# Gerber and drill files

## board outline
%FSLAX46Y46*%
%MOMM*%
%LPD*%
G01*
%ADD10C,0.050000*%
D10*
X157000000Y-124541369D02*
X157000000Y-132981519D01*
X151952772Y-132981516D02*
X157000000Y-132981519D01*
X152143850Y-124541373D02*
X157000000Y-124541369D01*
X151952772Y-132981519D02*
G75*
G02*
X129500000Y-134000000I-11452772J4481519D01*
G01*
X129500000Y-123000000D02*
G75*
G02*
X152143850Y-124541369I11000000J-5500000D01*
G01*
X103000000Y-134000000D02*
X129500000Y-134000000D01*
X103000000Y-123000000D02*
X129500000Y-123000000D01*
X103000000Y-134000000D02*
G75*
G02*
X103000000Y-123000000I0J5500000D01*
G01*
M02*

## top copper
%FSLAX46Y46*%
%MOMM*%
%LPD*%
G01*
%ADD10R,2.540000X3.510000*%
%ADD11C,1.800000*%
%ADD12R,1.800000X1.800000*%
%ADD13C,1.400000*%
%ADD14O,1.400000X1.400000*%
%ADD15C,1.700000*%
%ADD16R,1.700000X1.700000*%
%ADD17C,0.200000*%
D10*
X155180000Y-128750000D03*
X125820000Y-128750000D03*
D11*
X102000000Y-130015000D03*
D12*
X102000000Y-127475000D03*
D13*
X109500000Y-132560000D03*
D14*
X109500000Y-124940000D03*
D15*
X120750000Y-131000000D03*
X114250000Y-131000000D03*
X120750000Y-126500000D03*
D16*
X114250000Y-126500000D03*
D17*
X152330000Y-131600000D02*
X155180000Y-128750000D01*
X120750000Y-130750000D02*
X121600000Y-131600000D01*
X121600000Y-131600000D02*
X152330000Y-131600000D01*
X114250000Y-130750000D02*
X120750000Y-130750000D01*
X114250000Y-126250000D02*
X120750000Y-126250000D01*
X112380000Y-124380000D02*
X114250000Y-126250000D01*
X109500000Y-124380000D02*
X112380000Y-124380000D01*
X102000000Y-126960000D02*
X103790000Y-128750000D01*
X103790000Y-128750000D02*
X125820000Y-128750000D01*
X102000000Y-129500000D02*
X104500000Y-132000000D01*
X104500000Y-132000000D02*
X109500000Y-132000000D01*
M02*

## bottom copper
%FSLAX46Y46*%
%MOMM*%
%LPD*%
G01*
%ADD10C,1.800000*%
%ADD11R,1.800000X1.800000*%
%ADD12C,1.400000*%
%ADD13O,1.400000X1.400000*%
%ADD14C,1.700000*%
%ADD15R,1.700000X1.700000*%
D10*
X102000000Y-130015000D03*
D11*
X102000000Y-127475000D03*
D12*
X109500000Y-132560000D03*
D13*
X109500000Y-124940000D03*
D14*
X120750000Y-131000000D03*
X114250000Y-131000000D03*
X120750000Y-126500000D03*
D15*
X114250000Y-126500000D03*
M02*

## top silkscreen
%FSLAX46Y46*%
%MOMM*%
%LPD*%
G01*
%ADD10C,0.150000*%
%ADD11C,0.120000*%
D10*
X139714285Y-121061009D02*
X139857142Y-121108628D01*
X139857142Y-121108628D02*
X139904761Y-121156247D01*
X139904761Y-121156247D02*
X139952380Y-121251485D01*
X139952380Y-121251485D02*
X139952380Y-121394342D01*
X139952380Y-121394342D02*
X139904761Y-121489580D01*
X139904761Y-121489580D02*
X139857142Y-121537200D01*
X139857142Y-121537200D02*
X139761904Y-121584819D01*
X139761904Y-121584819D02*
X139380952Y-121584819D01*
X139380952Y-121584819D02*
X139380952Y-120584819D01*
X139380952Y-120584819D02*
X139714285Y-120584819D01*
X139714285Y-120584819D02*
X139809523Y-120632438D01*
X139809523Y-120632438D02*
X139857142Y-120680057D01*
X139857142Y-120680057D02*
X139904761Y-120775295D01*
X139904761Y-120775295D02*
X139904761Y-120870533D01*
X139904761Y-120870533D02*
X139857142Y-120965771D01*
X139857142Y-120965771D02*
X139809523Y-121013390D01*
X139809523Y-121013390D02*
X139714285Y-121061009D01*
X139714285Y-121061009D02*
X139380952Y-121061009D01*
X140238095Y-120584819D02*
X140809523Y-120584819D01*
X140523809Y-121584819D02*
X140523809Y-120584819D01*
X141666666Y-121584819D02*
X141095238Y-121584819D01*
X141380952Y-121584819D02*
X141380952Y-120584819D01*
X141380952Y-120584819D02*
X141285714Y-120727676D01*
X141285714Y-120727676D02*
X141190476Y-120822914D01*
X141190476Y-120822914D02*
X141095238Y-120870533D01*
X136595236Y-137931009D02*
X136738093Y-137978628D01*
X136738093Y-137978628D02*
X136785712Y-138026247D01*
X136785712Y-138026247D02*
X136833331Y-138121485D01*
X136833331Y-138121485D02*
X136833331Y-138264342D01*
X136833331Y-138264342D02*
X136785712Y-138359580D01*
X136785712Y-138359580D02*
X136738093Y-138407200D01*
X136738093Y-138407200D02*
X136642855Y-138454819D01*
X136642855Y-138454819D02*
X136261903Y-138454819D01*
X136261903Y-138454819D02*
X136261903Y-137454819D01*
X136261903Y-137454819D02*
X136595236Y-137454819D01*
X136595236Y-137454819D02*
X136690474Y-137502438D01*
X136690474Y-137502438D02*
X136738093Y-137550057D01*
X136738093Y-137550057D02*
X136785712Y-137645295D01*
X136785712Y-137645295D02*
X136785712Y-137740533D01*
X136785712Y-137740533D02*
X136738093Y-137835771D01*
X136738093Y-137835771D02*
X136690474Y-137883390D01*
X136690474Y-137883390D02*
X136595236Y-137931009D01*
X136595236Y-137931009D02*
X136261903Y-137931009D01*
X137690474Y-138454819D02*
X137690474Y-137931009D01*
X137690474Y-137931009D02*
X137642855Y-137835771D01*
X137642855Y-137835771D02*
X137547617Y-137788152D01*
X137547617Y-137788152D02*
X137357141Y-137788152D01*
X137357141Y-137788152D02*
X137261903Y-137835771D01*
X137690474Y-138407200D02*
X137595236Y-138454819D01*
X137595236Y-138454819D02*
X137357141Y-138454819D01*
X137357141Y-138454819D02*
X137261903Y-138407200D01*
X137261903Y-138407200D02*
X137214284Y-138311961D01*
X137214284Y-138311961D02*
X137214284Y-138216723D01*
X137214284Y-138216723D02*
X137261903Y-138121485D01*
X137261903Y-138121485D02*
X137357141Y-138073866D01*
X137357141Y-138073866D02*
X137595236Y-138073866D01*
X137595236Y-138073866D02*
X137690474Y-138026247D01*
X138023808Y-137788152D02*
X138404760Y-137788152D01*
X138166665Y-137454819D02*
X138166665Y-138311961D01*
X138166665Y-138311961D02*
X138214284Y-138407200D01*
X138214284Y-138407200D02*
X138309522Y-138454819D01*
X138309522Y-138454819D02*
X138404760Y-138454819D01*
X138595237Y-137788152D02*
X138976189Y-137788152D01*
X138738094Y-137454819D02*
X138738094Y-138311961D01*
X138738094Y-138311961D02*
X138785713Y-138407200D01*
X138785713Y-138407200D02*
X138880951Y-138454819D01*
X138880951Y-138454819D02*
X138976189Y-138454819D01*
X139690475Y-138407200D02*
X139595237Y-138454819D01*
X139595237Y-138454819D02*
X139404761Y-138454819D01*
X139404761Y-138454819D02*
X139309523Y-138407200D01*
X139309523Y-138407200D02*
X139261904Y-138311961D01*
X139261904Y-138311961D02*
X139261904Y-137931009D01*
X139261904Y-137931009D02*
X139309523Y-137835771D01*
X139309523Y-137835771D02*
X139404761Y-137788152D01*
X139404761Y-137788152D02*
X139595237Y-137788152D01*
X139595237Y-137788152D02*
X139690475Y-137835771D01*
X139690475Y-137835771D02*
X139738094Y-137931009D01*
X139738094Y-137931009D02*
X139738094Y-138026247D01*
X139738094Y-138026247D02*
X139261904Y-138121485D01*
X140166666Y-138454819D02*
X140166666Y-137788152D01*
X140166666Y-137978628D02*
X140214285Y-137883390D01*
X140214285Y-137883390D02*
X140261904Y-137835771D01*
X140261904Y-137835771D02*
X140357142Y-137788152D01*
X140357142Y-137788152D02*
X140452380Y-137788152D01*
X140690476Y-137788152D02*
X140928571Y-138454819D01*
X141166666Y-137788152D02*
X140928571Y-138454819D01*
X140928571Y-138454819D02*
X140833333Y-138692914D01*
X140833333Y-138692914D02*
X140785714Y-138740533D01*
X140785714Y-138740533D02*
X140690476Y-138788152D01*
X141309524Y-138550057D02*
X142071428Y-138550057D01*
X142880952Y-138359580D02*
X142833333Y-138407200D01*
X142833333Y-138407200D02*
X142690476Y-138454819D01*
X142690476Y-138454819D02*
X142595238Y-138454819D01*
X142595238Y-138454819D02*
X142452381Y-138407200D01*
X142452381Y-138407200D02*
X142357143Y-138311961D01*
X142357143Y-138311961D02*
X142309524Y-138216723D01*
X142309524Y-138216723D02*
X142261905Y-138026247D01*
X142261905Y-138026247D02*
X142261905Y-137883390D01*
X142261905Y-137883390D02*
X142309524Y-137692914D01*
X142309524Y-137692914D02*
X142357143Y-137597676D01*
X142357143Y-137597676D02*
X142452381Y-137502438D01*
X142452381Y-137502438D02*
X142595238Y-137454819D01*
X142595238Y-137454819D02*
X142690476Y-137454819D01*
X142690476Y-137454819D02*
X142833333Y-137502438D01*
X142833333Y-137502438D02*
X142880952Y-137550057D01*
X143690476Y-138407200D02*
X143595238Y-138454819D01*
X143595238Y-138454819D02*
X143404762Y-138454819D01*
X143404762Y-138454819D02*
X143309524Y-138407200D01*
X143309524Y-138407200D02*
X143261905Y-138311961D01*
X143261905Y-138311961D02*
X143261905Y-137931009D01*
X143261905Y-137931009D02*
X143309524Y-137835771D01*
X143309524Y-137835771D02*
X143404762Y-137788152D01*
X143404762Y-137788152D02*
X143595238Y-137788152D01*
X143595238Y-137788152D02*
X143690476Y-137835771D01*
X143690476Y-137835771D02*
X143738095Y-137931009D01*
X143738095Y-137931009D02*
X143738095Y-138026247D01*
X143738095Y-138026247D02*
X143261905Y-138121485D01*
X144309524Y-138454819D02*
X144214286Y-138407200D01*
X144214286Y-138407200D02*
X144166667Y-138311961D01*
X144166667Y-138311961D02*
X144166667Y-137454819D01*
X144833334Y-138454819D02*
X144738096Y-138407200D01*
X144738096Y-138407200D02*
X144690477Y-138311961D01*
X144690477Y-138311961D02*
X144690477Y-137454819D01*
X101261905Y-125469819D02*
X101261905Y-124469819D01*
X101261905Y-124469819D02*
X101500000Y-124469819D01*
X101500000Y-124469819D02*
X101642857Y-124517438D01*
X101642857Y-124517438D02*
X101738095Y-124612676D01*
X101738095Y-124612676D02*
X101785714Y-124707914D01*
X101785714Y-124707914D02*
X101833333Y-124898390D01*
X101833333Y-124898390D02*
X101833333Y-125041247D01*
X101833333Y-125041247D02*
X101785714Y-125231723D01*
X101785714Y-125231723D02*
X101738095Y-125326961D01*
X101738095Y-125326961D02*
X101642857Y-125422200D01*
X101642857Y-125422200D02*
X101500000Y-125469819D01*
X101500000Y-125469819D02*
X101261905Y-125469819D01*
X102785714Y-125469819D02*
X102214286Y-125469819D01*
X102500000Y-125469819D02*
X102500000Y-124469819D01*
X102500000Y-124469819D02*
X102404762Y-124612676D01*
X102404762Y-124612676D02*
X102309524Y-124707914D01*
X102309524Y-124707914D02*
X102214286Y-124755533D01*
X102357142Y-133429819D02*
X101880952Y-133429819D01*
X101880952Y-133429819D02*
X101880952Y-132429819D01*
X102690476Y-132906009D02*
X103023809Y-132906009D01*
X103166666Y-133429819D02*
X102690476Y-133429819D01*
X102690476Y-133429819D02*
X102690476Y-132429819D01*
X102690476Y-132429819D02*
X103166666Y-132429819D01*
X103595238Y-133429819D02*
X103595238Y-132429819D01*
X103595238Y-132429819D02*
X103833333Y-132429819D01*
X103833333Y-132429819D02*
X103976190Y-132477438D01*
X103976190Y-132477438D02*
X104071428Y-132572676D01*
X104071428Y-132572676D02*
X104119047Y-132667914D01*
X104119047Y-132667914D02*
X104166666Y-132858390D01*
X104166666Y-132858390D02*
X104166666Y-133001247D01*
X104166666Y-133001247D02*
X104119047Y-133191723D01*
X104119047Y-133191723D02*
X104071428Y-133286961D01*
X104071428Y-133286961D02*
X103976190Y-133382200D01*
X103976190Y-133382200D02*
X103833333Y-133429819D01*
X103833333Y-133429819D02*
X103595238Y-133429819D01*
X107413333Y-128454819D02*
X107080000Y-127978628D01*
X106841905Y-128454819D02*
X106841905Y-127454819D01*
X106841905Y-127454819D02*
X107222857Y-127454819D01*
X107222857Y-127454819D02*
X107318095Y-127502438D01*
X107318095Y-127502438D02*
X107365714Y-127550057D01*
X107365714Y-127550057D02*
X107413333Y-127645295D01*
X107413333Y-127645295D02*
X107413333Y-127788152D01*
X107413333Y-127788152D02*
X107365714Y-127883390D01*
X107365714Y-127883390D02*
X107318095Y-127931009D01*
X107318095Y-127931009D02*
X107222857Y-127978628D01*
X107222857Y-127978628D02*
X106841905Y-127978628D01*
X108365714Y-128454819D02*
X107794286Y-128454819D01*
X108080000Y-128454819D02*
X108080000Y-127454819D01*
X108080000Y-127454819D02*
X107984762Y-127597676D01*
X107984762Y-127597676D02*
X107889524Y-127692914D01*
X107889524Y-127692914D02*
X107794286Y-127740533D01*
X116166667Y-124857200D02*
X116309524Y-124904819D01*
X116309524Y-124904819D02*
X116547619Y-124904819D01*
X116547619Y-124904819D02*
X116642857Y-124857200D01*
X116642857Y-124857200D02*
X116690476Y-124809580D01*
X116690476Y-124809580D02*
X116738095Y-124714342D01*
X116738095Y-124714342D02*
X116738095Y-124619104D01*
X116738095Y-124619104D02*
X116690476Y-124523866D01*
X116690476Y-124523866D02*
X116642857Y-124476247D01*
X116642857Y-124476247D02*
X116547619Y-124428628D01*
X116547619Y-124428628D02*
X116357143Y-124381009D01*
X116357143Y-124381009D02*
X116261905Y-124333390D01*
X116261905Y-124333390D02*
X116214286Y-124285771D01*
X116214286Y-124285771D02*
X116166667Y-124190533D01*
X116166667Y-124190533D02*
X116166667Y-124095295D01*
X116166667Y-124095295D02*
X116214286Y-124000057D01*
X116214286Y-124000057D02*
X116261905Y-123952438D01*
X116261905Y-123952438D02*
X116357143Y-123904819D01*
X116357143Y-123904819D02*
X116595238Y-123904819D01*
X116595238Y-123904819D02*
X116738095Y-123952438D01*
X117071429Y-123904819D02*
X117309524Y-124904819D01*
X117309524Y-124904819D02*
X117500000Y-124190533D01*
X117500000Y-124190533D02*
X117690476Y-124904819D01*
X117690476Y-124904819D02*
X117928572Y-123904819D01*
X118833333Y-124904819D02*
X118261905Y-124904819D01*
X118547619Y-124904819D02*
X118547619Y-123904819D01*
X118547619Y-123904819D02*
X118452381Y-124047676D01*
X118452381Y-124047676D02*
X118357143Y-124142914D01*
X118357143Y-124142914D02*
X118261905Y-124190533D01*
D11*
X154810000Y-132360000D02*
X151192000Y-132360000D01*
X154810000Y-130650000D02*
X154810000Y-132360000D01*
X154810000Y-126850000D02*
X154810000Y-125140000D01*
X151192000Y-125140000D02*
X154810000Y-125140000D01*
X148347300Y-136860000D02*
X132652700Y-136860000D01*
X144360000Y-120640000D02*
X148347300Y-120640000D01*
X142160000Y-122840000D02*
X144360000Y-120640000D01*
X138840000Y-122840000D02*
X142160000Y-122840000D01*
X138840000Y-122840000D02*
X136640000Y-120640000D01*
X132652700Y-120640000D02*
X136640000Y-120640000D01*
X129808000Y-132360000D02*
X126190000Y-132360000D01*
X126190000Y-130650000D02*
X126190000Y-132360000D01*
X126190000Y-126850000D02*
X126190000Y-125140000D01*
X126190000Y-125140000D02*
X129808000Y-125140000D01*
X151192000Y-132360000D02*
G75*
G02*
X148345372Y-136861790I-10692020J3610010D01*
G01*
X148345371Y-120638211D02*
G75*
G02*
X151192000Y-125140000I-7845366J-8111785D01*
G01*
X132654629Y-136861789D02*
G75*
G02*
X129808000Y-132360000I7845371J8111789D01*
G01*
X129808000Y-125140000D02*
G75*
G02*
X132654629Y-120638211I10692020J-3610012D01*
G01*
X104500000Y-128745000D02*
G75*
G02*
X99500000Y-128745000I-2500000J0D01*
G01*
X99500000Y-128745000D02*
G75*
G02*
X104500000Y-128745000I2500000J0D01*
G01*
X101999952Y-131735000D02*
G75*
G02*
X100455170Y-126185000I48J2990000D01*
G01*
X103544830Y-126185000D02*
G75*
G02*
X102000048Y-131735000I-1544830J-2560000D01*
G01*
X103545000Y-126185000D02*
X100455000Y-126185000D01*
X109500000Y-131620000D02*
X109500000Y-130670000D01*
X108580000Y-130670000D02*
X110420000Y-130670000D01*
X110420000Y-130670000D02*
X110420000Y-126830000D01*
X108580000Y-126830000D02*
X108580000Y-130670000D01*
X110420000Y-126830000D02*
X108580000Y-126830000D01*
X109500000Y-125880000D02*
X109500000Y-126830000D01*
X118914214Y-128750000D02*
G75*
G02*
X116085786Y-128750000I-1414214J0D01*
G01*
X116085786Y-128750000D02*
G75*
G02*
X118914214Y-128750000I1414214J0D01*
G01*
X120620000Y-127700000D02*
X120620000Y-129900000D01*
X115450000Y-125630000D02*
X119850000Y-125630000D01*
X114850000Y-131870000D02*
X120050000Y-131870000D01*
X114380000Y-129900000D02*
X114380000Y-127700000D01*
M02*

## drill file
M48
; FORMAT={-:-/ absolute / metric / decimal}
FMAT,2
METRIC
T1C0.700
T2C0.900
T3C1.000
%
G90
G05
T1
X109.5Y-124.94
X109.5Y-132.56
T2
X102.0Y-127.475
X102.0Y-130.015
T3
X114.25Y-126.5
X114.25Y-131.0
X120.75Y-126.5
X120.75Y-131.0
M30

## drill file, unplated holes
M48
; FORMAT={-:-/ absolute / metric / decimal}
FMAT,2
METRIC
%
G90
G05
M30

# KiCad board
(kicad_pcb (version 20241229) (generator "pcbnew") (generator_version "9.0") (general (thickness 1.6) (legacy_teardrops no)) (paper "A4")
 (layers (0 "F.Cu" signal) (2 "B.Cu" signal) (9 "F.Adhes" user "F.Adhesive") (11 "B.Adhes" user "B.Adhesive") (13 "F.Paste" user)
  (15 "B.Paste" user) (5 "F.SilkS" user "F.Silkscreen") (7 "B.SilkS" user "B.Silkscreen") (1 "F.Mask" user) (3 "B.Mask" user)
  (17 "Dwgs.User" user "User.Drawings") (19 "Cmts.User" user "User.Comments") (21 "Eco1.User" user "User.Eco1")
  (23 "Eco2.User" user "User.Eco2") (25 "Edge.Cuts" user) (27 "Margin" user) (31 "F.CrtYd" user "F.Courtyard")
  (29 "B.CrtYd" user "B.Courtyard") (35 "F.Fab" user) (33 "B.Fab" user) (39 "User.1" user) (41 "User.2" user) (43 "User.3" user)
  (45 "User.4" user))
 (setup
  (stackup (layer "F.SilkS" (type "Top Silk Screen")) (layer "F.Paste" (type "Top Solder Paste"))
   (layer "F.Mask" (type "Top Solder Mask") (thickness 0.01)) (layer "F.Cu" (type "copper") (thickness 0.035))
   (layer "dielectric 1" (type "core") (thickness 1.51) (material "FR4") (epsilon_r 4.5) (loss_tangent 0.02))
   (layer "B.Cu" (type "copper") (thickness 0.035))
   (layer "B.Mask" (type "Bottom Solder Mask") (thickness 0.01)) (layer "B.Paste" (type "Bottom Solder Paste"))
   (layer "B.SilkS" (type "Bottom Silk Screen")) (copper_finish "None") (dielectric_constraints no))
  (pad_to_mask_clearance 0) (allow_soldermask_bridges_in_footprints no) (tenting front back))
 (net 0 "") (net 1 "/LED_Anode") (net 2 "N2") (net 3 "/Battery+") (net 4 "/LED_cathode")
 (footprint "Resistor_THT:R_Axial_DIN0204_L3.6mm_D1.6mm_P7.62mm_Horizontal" (layer "F.Cu") (at 109.5 132.56 90)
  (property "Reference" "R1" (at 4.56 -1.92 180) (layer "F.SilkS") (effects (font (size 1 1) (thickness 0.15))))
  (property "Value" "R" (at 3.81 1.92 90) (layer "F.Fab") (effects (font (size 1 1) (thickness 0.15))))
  (fp_line (start 5.73 -0.92) (end 1.89 -0.92) (stroke (width 0.12) (type solid)) (layer "F.SilkS"))
  (fp_line (start 1.89 -0.92) (end 1.89 0.92) (stroke (width 0.12) (type solid)) (layer "F.SilkS"))
  (fp_line (start 6.68 0) (end 5.73 0) (stroke (width 0.12) (type solid)) (layer "F.SilkS"))
  (fp_line (start 0.94 0) (end 1.89 0) (stroke (width 0.12) (type solid)) (layer "F.SilkS"))
  (fp_line (start 5.73 0.92) (end 5.73 -0.92) (stroke (width 0.12) (type solid)) (layer "F.SilkS"))
  (fp_line (start 1.89 0.92) (end 5.73 0.92) (stroke (width 0.12) (type solid)) (layer "F.SilkS"))
  (pad "1" thru_hole circle (at 0 0 90) (size 1.4 1.4) (drill 0.7) (layers "*.Cu" "*.Mask") (remove_unused_layers no) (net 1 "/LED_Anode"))
  (pad "2" thru_hole oval (at 7.62 0 90) (size 1.4 1.4) (drill 0.7) (layers "*.Cu" "*.Mask") (remove_unused_layers no) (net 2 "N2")))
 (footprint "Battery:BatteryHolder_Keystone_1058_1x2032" (layer "F.Cu") (at 140.5 128.75 180)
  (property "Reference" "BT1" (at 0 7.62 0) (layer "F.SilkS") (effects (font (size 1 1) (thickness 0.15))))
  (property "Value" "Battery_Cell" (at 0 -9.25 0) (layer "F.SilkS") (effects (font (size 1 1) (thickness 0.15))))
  (fp_line (start 14.31 3.61) (end 10.692 3.61) (stroke (width 0.12) (type solid)) (layer "F.SilkS"))
  (fp_line (start 14.31 1.9) (end 14.31 3.61) (stroke (width 0.12) (type solid)) (layer "F.SilkS"))
  (fp_line (start 14.31 -1.9) (end 14.31 -3.61) (stroke (width 0.12) (type solid)) (layer "F.SilkS"))
  (fp_line (start 10.692 -3.61) (end 14.31 -3.61) (stroke (width 0.12) (type solid)) (layer "F.SilkS"))
  (fp_line (start 7.8473 8.11) (end 3.86 8.11) (stroke (width 0.12) (type solid)) (layer "F.SilkS"))
  (fp_line (start 1.66 5.91) (end 3.86 8.11) (stroke (width 0.12) (type solid)) (layer "F.SilkS"))
  (fp_line (start 1.66 5.91) (end -1.66 5.91) (stroke (width 0.12) (type solid)) (layer "F.SilkS"))
  (fp_line (start -1.66 5.91) (end -3.86 8.11) (stroke (width 0.12) (type solid)) (layer "F.SilkS"))
  (fp_line (start -3.86 8.11) (end -7.8473 8.11) (stroke (width 0.12) (type solid)) (layer "F.SilkS"))
  (fp_line (start -7.8473 -8.11) (end 7.8473 -8.11) (stroke (width 0.12) (type solid)) (layer "F.SilkS"))
  (fp_line (start -10.692 3.61) (end -14.31 3.61) (stroke (width 0.12) (type solid)) (layer "F.SilkS"))
  (fp_line (start -14.31 1.9) (end -14.31 3.61) (stroke (width 0.12) (type solid)) (layer "F.SilkS"))
  (fp_line (start -14.31 -1.9) (end -14.31 -3.61) (stroke (width 0.12) (type solid)) (layer "F.SilkS"))
  (fp_line (start -14.31 -3.61) (end -10.692 -3.61) (stroke (width 0.12) (type solid)) (layer "F.SilkS"))
  (fp_arc (start 10.692 3.61) (mid 9.538084 6.031244) (end 7.845371 8.111789) (stroke (width 0.12) (type solid)) (layer "F.SilkS"))
  (fp_arc (start 7.845371 -8.111789) (mid 9.538085 -6.031244) (end 10.692 -3.61) (stroke (width 0.12) (type solid)) (layer "F.SilkS"))
  (fp_arc (start -7.845371 8.111789) (mid -9.538085 6.031244) (end -10.692 3.61) (stroke (width 0.12) (type solid)) (layer "F.SilkS"))
  (fp_arc (start -10.692 -3.61) (mid -9.538084 -6.031244) (end -7.845371 -8.111789) (stroke (width 0.12) (type solid)) (layer "F.SilkS"))
  (pad "1" smd rect (at -14.68 0 180) (size 2.54 3.51) (layers "F.Cu" "F.Mask" "F.Paste") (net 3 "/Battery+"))
  (pad "2" smd rect (at 14.68 0 180) (size 2.54 3.51) (layers "F.Cu" "F.Mask" "F.Paste") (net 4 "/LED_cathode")))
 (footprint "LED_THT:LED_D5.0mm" (layer "F.Cu") (at 102 127.475 -90)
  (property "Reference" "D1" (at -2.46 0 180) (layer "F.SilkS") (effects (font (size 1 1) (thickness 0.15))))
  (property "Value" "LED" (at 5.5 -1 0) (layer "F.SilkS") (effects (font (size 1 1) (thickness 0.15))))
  (fp_line (start -1.29 -1.545) (end -1.29 1.545) (stroke (width 0.12) (type solid)) (layer "F.SilkS"))
  (fp_arc (start 4.26 0.000048) (mid 2.071756 2.880501) (end -1.29 1.54483) (stroke (width 0.12) (type solid)) (layer "F.SilkS"))
  (fp_arc (start -1.29 -1.54483) (mid 2.071756 -2.880501) (end 4.26 -0.000048) (stroke (width 0.12) (type solid)) (layer "F.SilkS"))
  (fp_circle (center 1.27 0) (end 3.77 0) (stroke (width 0.12) (type solid)) (fill no) (layer "F.SilkS"))
  (pad "1" thru_hole rect (at 0 0 270) (size 1.8 1.8) (drill 0.9) (layers "*.Cu" "*.Mask") (remove_unused_layers no) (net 4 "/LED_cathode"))
  (pad "2" thru_hole circle (at 2.54 0 270) (size 1.8 1.8) (drill 0.9) (layers "*.Cu" "*.Mask") (remove_unused_layers no)
   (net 1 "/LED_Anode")))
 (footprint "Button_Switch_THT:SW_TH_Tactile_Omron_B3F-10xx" (layer "F.Cu") (at 114.25 126.5)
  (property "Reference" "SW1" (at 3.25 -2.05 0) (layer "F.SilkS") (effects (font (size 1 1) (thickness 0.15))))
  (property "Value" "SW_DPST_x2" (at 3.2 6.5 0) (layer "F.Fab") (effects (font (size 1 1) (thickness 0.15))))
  (fp_line (start 0.13 3.4) (end 0.13 1.2) (stroke (width 0.12) (type solid)) (layer "F.SilkS"))
  (fp_line (start 0.6 5.37) (end 5.8 5.37) (stroke (width 0.12) (type solid)) (layer "F.SilkS"))
  (fp_line (start 1.2 -0.87) (end 5.6 -0.87) (stroke (width 0.12) (type solid)) (layer "F.SilkS"))
  (fp_line (start 6.37 1.2) (end 6.37 3.4) (stroke (width 0.12) (type solid)) (layer "F.SilkS"))
  (fp_circle (center 3.25 2.25) (end 4.25 3.25) (stroke (width 0.12) (type solid)) (fill no) (layer "F.SilkS"))
  (pad "1" thru_hole rect (at 0 0) (size 1.7 1.7) (drill 1) (layers "*.Cu" "*.Mask") (remove_unused_layers no) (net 2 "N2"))
  (pad "1" thru_hole circle (at 6.5 0) (size 1.7 1.7) (drill 1) (layers "*.Cu" "*.Mask") (remove_unused_layers no) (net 2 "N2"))
  (pad "2" thru_hole circle (at 0 4.5) (size 1.7 1.7) (drill 1) (layers "*.Cu" "*.Mask") (remove_unused_layers no) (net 3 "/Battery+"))
  (pad "2" thru_hole circle (at 6.5 4.5) (size 1.7 1.7) (drill 1) (layers "*.Cu" "*.Mask") (remove_unused_layers no) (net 3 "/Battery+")))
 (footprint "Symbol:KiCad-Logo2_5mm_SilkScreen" (layer "B.Cu") (at 140.5 126 180)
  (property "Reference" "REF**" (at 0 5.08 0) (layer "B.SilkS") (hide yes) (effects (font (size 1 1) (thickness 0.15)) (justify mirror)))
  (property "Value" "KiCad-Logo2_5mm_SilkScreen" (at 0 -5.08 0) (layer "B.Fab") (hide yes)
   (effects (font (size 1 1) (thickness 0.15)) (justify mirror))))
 (gr_line (start 103 134) (end 129.5 134) (stroke (width 0.05) (type default)) (locked yes) (layer "Edge.Cuts"))
 (gr_line (start 103 123) (end 129.5 123) (stroke (width 0.05) (type default)) (locked yes) (layer "Edge.Cuts"))
 (gr_line (start 157 124.541369) (end 157 132.981519) (stroke (width 0.05) (type default)) (locked yes) (layer "Edge.Cuts"))
 (gr_line (start 151.952772 132.981516) (end 157 132.981519) (stroke (width 0.05) (type default)) (locked yes) (layer "Edge.Cuts"))
 (gr_arc (start 103 134) (mid 97.5 128.5) (end 103 123) (stroke (width 0.05) (type default)) (locked yes) (layer "Edge.Cuts"))
 (gr_line (start 152.14385 124.541373) (end 157 124.541369) (stroke (width 0.05) (type default)) (locked yes) (layer "Edge.Cuts"))
 (gr_arc (start 151.952772 132.981519) (mid 141.057294 140.785741) (end 129.5 134) (stroke (width 0.05) (type default)) (locked yes)
  (layer "Edge.Cuts"))
 (gr_arc (start 129.5 123) (mid 141.335219 116.23002) (end 152.14385 124.541369) (stroke (width 0.05) (type default)) (locked yes)
  (layer "Edge.Cuts"))
 (segment (start 121.6 131.6) (end 152.33 131.6) (width 0.2) (layer "F.Cu") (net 3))
 (segment (start 120.75 130.75) (end 121.6 131.6) (width 0.2) (layer "F.Cu") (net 3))
 (segment (start 152.33 131.6) (end 155.18 128.75) (width 0.2) (layer "F.Cu") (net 3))
 (segment (start 114.25 130.75) (end 120.75 130.75) (width 0.2) (layer "F.Cu") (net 3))
 (segment (start 102 126.96) (end 103.79 128.75) (width 0.2) (layer "F.Cu") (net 4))
 (segment (start 103.79 128.75) (end 125.82 128.75) (width 0.2) (layer "F.Cu") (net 4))
 (segment (start 102 129.5) (end 104.5 132) (width 0.2) (layer "F.Cu") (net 1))
 (segment (start 104.5 132) (end 109.5 132) (width 0.2) (layer "F.Cu") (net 1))
 (segment (start 112.38 124.38) (end 114.25 126.25) (width 0.2) (layer "F.Cu") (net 2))
 (segment (start 109.5 124.38) (end 112.38 124.38) (width 0.2) (layer "F.Cu") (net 2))
 (segment (start 114.25 126.25) (end 120.75 126.25) (width 0.2) (layer "F.Cu") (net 2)))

